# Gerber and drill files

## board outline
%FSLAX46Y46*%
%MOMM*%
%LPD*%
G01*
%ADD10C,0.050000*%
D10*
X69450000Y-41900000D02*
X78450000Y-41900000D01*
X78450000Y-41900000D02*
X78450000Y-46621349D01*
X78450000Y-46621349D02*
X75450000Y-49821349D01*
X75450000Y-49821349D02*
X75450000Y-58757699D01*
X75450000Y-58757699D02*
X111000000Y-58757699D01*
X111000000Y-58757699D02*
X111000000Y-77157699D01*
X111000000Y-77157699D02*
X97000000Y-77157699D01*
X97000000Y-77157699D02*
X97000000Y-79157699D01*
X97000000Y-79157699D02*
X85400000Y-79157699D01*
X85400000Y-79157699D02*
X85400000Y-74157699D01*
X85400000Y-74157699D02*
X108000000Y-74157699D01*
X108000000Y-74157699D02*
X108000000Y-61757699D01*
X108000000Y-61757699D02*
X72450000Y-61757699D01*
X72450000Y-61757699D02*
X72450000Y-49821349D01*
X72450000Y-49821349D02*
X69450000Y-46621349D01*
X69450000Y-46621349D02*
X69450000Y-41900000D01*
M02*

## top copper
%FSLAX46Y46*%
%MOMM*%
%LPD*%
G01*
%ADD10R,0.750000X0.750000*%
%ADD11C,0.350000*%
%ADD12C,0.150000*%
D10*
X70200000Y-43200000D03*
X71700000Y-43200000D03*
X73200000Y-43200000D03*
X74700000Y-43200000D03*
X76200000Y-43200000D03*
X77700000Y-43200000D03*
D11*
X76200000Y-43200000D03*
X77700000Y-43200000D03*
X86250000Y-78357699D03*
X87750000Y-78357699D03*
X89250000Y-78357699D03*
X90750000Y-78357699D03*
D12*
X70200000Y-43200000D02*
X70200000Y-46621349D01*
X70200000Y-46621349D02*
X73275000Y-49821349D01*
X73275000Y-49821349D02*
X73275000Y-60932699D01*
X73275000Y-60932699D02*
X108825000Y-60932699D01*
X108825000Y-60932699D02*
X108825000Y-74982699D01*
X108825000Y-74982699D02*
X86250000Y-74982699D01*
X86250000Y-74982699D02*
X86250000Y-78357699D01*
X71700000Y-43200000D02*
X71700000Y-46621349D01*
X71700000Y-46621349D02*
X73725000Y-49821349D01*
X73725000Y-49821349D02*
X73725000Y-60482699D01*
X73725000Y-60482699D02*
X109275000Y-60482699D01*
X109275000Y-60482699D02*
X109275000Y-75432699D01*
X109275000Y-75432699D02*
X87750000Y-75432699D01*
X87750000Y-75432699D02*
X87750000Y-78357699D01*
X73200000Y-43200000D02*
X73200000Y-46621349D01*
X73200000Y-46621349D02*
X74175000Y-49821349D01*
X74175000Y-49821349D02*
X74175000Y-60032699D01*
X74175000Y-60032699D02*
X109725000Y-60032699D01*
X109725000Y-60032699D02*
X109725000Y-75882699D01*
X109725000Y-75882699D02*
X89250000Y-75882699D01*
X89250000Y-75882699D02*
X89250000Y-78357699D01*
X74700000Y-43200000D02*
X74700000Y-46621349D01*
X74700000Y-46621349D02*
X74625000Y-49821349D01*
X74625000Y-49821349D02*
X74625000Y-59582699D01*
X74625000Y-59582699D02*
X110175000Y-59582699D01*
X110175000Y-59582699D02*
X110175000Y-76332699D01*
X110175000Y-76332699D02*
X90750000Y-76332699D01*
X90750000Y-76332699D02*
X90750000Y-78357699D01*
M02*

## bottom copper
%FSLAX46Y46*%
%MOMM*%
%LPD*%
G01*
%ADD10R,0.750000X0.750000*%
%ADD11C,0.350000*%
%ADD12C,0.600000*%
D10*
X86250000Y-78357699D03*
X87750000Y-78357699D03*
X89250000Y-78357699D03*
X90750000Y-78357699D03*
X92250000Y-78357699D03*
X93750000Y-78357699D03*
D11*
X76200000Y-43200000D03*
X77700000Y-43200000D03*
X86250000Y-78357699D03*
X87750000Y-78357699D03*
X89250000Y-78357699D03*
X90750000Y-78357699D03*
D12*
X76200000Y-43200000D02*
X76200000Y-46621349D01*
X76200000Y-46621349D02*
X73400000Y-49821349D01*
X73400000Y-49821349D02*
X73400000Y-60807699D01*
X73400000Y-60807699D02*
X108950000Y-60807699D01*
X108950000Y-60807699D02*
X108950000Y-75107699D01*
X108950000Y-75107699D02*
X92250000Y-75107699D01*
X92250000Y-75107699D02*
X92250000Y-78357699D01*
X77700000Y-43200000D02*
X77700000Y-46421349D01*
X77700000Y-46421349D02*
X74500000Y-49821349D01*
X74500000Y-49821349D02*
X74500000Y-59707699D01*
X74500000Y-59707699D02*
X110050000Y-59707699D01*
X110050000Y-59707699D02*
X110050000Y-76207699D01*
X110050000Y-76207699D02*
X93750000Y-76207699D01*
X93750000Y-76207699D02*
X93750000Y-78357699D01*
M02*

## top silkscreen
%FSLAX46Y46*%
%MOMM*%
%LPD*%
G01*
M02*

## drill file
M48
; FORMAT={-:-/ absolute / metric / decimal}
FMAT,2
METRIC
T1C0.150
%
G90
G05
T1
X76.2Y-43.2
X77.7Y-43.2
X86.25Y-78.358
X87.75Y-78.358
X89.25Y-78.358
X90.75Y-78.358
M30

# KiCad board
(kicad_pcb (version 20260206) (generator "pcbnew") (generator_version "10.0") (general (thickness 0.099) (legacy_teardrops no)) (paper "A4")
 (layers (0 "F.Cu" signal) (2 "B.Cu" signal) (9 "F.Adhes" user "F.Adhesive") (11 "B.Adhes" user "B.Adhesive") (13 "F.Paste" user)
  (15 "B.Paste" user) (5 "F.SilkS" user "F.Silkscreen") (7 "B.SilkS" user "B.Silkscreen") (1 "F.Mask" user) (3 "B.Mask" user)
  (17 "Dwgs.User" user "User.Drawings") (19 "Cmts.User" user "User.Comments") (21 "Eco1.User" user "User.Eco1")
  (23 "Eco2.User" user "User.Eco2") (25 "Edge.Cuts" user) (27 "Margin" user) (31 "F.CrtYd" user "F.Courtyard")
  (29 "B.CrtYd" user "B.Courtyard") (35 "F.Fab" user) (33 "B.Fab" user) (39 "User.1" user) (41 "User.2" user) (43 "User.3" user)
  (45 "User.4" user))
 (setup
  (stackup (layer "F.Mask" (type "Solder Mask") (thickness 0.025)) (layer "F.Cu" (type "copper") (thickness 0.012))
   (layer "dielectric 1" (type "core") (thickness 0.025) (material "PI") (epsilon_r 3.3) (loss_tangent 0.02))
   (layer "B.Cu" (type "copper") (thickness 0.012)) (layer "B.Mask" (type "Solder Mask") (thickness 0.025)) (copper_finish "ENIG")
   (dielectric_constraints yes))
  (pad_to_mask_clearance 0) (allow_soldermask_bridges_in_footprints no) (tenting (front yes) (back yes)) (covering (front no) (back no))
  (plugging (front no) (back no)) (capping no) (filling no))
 (gr_line (start 69.45 41.90000000000001) (end 78.45 41.90000000000001) (stroke (width 0.05) (type default)) (layer "Edge.Cuts"))
 (gr_line (start 78.45 41.90000000000001) (end 78.45 46.62134939012759) (stroke (width 0.05) (type default)) (layer "Edge.Cuts"))
 (gr_line (start 78.45 46.62134939012759) (end 75.45 49.821349390127594) (stroke (width 0.05) (type default)) (layer "Edge.Cuts"))
 (gr_line (start 75.45 49.821349390127594) (end 75.45 58.75769878025519) (stroke (width 0.05) (type default)) (layer "Edge.Cuts"))
 (gr_line (start 75.45 58.75769878025519) (end 111.0 58.75769878025519) (stroke (width 0.05) (type default)) (layer "Edge.Cuts"))
 (gr_line (start 111.0 58.75769878025519) (end 111.0 77.15769878025519) (stroke (width 0.05) (type default)) (layer "Edge.Cuts"))
 (gr_line (start 111.0 77.15769878025519) (end 97.0 77.15769878025519) (stroke (width 0.05) (type default)) (layer "Edge.Cuts"))
 (gr_line (start 97.0 77.15769878025519) (end 97.0 79.15769878025519) (stroke (width 0.05) (type default)) (layer "Edge.Cuts"))
 (gr_line (start 97.0 79.15769878025519) (end 85.4 79.15769878025519) (stroke (width 0.05) (type default)) (layer "Edge.Cuts"))
 (gr_line (start 85.4 79.15769878025519) (end 85.4 74.15769878025519) (stroke (width 0.05) (type default)) (layer "Edge.Cuts"))
 (gr_line (start 85.4 74.15769878025519) (end 108.0 74.15769878025519) (stroke (width 0.05) (type default)) (layer "Edge.Cuts"))
 (gr_line (start 108.0 74.15769878025519) (end 108.0 61.75769878025519) (stroke (width 0.05) (type default)) (layer "Edge.Cuts"))
 (gr_line (start 108.0 61.75769878025519) (end 72.45 61.75769878025519) (stroke (width 0.05) (type default)) (layer "Edge.Cuts"))
 (gr_line (start 72.45 61.75769878025519) (end 72.45 49.821349390127594) (stroke (width 0.05) (type default)) (layer "Edge.Cuts"))
 (gr_line (start 72.45 49.821349390127594) (end 69.45 46.62134939012759) (stroke (width 0.05) (type default)) (layer "Edge.Cuts"))
 (gr_line (start 69.45 46.62134939012759) (end 69.45 41.90000000000001) (stroke (width 0.05) (type default)) (layer "Edge.Cuts"))
 (via (at 76.2 43.2) (size 0.35) (drill 0.15) (layers "F.Cu" "B.Cu") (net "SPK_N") (locked yes))
 (via (at 77.7 43.2) (size 0.35) (drill 0.15) (layers "F.Cu" "B.Cu") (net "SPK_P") (locked yes))
 (via (at 86.25 78.35769878025519) (size 0.35) (drill 0.15) (layers "F.Cu" "B.Cu") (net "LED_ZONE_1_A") (locked yes))
 (via (at 87.75 78.35769878025519) (size 0.35) (drill 0.15) (layers "F.Cu" "B.Cu") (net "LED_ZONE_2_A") (locked yes))
 (via (at 89.25 78.35769878025519) (size 0.35) (drill 0.15) (layers "F.Cu" "B.Cu") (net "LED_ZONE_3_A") (locked yes))
 (via (at 90.75 78.35769878025519) (size 0.35) (drill 0.15) (layers "F.Cu" "B.Cu") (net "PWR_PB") (locked yes))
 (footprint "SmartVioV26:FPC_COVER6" (layer "F.Cu") (at 0 0)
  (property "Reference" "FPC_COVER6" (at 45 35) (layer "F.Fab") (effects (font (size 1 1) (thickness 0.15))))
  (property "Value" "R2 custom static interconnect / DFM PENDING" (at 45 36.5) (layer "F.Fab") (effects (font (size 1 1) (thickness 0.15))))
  (pad "S1" smd rect (at 70.2 43.2) (size 0.75 0.75) (layers "F.Cu" "F.Mask") (solder_mask_margin 0.1) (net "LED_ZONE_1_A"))
  (pad "S2" smd rect (at 71.7 43.2) (size 0.75 0.75) (layers "F.Cu" "F.Mask") (solder_mask_margin 0.1) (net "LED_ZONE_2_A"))
  (pad "S3" smd rect (at 73.2 43.2) (size 0.75 0.75) (layers "F.Cu" "F.Mask") (solder_mask_margin 0.1) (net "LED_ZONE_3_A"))
  (pad "S4" smd rect (at 74.7 43.2) (size 0.75 0.75) (layers "F.Cu" "F.Mask") (solder_mask_margin 0.1) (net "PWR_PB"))
  (pad "S5" smd rect (at 76.2 43.2) (size 0.75 0.75) (layers "F.Cu" "F.Mask") (solder_mask_margin 0.1) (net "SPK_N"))
  (pad "S6" smd rect (at 77.7 43.2) (size 0.75 0.75) (layers "F.Cu" "F.Mask") (solder_mask_margin 0.1) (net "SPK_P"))
  (pad "T1" smd rect (at 86.25 78.35769878025519) (size 0.75 0.75) (layers "B.Cu" "B.Mask") (solder_mask_margin 0.1) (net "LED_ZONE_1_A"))
  (pad "T2" smd rect (at 87.75 78.35769878025519) (size 0.75 0.75) (layers "B.Cu" "B.Mask") (solder_mask_margin 0.1) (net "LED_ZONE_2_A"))
  (pad "T3" smd rect (at 89.25 78.35769878025519) (size 0.75 0.75) (layers "B.Cu" "B.Mask") (solder_mask_margin 0.1) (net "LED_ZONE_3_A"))
  (pad "T4" smd rect (at 90.75 78.35769878025519) (size 0.75 0.75) (layers "B.Cu" "B.Mask") (solder_mask_margin 0.1) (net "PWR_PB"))
  (pad "T5" smd rect (at 92.25 78.35769878025519) (size 0.75 0.75) (layers "B.Cu" "B.Mask") (solder_mask_margin 0.1) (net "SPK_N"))
  (pad "T6" smd rect (at 93.75 78.35769878025519) (size 0.75 0.75) (layers "B.Cu" "B.Mask") (solder_mask_margin 0.1) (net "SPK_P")))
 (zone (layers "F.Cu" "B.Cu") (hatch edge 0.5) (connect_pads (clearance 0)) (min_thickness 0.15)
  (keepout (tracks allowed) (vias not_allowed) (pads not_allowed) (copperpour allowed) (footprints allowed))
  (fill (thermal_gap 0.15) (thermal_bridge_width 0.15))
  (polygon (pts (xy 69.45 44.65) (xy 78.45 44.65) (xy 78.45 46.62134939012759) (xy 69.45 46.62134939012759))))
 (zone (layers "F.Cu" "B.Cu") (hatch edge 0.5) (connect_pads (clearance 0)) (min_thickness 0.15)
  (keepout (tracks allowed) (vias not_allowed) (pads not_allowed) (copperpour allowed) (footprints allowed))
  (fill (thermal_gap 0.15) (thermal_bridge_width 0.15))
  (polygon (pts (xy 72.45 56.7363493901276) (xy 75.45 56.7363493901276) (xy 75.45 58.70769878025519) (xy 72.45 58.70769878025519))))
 (segment (start 70.2 43.2) (end 70.2 46.62134939012759) (width 0.15) (layer "F.Cu") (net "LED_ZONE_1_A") (locked yes))
 (segment (start 70.2 46.62134939012759) (end 73.275 49.821349390127594) (width 0.15) (layer "F.Cu") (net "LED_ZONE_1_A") (locked yes))
 (segment (start 73.275 49.821349390127594) (end 73.275 60.93269878025519) (width 0.15) (layer "F.Cu") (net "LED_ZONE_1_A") (locked yes))
 (segment (start 73.275 60.93269878025519) (end 108.825 60.93269878025519) (width 0.15) (layer "F.Cu") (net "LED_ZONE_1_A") (locked yes))
 (segment (start 108.825 60.93269878025519) (end 108.825 74.98269878025519) (width 0.15) (layer "F.Cu") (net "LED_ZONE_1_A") (locked yes))
 (segment (start 108.825 74.98269878025519) (end 86.25 74.98269878025519) (width 0.15) (layer "F.Cu") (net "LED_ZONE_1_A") (locked yes))
 (segment (start 86.25 74.98269878025519) (end 86.25 78.35769878025519) (width 0.15) (layer "F.Cu") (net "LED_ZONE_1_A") (locked yes))
 (segment (start 71.7 43.2) (end 71.7 46.62134939012759) (width 0.15) (layer "F.Cu") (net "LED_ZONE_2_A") (locked yes))
 (segment (start 71.7 46.62134939012759) (end 73.72500000000001 49.821349390127594) (width 0.15) (layer "F.Cu") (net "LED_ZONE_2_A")
  (locked yes))
 (segment (start 73.72500000000001 49.821349390127594) (end 73.72500000000001 60.48269878025519) (width 0.15) (layer "F.Cu")
  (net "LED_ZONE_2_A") (locked yes))
 (segment (start 73.72500000000001 60.48269878025519) (end 109.275 60.48269878025519) (width 0.15) (layer "F.Cu") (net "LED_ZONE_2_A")
  (locked yes))
 (segment (start 109.275 60.48269878025519) (end 109.275 75.4326987802552) (width 0.15) (layer "F.Cu") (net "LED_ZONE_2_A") (locked yes))
 (segment (start 109.275 75.4326987802552) (end 87.75 75.4326987802552) (width 0.15) (layer "F.Cu") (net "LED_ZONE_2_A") (locked yes))
 (segment (start 87.75 75.4326987802552) (end 87.75 78.35769878025519) (width 0.15) (layer "F.Cu") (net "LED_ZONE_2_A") (locked yes))
 (segment (start 73.2 43.2) (end 73.2 46.62134939012759) (width 0.15) (layer "F.Cu") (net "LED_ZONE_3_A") (locked yes))
 (segment (start 73.2 46.62134939012759) (end 74.175 49.821349390127594) (width 0.15) (layer "F.Cu") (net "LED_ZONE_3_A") (locked yes))
 (segment (start 74.175 49.821349390127594) (end 74.175 60.03269878025519) (width 0.15) (layer "F.Cu") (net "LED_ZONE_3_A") (locked yes))
 (segment (start 74.175 60.03269878025519) (end 109.725 60.03269878025519) (width 0.15) (layer "F.Cu") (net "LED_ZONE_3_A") (locked yes))
 (segment (start 109.725 60.03269878025519) (end 109.725 75.88269878025518) (width 0.15) (layer "F.Cu") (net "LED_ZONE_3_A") (locked yes))
 (segment (start 109.725 75.88269878025518) (end 89.25 75.88269878025518) (width 0.15) (layer "F.Cu") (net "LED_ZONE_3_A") (locked yes))
 (segment (start 89.25 75.88269878025518) (end 89.25 78.35769878025519) (width 0.15) (layer "F.Cu") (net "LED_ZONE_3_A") (locked yes))
 (segment (start 74.7 43.2) (end 74.7 46.62134939012759) (width 0.15) (layer "F.Cu") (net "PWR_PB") (locked yes))
 (segment (start 74.7 46.62134939012759) (end 74.625 49.821349390127594) (width 0.15) (layer "F.Cu") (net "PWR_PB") (locked yes))
 (segment (start 74.625 49.821349390127594) (end 74.625 59.58269878025519) (width 0.15) (layer "F.Cu") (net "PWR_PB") (locked yes))
 (segment (start 74.625 59.58269878025519) (end 110.175 59.58269878025519) (width 0.15) (layer "F.Cu") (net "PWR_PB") (locked yes))
 (segment (start 110.175 59.58269878025519) (end 110.175 76.33269878025519) (width 0.15) (layer "F.Cu") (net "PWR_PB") (locked yes))
 (segment (start 110.175 76.33269878025519) (end 90.75 76.33269878025519) (width 0.15) (layer "F.Cu") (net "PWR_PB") (locked yes))
 (segment (start 90.75 76.33269878025519) (end 90.75 78.35769878025519) (width 0.15) (layer "F.Cu") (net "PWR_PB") (locked yes))
 (segment (start 76.2 43.2) (end 76.2 46.62134939012759) (width 0.6) (layer "B.Cu") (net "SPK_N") (locked yes))
 (segment (start 76.2 46.62134939012759) (end 73.4 49.821349390127594) (width 0.6) (layer "B.Cu") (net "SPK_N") (locked yes))
 (segment (start 73.4 49.821349390127594) (end 73.4 60.80769878025519) (width 0.6) (layer "B.Cu") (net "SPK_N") (locked yes))
 (segment (start 73.4 60.80769878025519) (end 108.95 60.80769878025519) (width 0.6) (layer "B.Cu") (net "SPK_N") (locked yes))
 (segment (start 108.95 60.80769878025519) (end 108.95 75.10769878025519) (width 0.6) (layer "B.Cu") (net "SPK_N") (locked yes))
 (segment (start 108.95 75.10769878025519) (end 92.25 75.10769878025519) (width 0.6) (layer "B.Cu") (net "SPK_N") (locked yes))
 (segment (start 92.25 75.10769878025519) (end 92.25 78.35769878025519) (width 0.6) (layer "B.Cu") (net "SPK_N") (locked yes))
 (segment (start 77.7 43.2) (end 77.7 46.42134939012759) (width 0.6) (layer "B.Cu") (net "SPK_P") (locked yes))
 (segment (start 77.7 46.42134939012759) (end 74.5 49.821349390127594) (width 0.6) (layer "B.Cu") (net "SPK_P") (locked yes))
 (segment (start 74.5 49.821349390127594) (end 74.5 59.70769878025519) (width 0.6) (layer "B.Cu") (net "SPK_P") (locked yes))
 (segment (start 74.5 59.70769878025519) (end 110.05 59.70769878025519) (width 0.6) (layer "B.Cu") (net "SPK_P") (locked yes))
 (segment (start 110.05 59.70769878025519) (end 110.05 76.20769878025519) (width 0.6) (layer "B.Cu") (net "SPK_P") (locked yes))
 (segment (start 110.05 76.20769878025519) (end 93.75 76.20769878025519) (width 0.6) (layer "B.Cu") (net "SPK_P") (locked yes))
 (segment (start 93.75 76.20769878025519) (end 93.75 78.35769878025519) (width 0.6) (layer "B.Cu") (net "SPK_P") (locked yes)))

